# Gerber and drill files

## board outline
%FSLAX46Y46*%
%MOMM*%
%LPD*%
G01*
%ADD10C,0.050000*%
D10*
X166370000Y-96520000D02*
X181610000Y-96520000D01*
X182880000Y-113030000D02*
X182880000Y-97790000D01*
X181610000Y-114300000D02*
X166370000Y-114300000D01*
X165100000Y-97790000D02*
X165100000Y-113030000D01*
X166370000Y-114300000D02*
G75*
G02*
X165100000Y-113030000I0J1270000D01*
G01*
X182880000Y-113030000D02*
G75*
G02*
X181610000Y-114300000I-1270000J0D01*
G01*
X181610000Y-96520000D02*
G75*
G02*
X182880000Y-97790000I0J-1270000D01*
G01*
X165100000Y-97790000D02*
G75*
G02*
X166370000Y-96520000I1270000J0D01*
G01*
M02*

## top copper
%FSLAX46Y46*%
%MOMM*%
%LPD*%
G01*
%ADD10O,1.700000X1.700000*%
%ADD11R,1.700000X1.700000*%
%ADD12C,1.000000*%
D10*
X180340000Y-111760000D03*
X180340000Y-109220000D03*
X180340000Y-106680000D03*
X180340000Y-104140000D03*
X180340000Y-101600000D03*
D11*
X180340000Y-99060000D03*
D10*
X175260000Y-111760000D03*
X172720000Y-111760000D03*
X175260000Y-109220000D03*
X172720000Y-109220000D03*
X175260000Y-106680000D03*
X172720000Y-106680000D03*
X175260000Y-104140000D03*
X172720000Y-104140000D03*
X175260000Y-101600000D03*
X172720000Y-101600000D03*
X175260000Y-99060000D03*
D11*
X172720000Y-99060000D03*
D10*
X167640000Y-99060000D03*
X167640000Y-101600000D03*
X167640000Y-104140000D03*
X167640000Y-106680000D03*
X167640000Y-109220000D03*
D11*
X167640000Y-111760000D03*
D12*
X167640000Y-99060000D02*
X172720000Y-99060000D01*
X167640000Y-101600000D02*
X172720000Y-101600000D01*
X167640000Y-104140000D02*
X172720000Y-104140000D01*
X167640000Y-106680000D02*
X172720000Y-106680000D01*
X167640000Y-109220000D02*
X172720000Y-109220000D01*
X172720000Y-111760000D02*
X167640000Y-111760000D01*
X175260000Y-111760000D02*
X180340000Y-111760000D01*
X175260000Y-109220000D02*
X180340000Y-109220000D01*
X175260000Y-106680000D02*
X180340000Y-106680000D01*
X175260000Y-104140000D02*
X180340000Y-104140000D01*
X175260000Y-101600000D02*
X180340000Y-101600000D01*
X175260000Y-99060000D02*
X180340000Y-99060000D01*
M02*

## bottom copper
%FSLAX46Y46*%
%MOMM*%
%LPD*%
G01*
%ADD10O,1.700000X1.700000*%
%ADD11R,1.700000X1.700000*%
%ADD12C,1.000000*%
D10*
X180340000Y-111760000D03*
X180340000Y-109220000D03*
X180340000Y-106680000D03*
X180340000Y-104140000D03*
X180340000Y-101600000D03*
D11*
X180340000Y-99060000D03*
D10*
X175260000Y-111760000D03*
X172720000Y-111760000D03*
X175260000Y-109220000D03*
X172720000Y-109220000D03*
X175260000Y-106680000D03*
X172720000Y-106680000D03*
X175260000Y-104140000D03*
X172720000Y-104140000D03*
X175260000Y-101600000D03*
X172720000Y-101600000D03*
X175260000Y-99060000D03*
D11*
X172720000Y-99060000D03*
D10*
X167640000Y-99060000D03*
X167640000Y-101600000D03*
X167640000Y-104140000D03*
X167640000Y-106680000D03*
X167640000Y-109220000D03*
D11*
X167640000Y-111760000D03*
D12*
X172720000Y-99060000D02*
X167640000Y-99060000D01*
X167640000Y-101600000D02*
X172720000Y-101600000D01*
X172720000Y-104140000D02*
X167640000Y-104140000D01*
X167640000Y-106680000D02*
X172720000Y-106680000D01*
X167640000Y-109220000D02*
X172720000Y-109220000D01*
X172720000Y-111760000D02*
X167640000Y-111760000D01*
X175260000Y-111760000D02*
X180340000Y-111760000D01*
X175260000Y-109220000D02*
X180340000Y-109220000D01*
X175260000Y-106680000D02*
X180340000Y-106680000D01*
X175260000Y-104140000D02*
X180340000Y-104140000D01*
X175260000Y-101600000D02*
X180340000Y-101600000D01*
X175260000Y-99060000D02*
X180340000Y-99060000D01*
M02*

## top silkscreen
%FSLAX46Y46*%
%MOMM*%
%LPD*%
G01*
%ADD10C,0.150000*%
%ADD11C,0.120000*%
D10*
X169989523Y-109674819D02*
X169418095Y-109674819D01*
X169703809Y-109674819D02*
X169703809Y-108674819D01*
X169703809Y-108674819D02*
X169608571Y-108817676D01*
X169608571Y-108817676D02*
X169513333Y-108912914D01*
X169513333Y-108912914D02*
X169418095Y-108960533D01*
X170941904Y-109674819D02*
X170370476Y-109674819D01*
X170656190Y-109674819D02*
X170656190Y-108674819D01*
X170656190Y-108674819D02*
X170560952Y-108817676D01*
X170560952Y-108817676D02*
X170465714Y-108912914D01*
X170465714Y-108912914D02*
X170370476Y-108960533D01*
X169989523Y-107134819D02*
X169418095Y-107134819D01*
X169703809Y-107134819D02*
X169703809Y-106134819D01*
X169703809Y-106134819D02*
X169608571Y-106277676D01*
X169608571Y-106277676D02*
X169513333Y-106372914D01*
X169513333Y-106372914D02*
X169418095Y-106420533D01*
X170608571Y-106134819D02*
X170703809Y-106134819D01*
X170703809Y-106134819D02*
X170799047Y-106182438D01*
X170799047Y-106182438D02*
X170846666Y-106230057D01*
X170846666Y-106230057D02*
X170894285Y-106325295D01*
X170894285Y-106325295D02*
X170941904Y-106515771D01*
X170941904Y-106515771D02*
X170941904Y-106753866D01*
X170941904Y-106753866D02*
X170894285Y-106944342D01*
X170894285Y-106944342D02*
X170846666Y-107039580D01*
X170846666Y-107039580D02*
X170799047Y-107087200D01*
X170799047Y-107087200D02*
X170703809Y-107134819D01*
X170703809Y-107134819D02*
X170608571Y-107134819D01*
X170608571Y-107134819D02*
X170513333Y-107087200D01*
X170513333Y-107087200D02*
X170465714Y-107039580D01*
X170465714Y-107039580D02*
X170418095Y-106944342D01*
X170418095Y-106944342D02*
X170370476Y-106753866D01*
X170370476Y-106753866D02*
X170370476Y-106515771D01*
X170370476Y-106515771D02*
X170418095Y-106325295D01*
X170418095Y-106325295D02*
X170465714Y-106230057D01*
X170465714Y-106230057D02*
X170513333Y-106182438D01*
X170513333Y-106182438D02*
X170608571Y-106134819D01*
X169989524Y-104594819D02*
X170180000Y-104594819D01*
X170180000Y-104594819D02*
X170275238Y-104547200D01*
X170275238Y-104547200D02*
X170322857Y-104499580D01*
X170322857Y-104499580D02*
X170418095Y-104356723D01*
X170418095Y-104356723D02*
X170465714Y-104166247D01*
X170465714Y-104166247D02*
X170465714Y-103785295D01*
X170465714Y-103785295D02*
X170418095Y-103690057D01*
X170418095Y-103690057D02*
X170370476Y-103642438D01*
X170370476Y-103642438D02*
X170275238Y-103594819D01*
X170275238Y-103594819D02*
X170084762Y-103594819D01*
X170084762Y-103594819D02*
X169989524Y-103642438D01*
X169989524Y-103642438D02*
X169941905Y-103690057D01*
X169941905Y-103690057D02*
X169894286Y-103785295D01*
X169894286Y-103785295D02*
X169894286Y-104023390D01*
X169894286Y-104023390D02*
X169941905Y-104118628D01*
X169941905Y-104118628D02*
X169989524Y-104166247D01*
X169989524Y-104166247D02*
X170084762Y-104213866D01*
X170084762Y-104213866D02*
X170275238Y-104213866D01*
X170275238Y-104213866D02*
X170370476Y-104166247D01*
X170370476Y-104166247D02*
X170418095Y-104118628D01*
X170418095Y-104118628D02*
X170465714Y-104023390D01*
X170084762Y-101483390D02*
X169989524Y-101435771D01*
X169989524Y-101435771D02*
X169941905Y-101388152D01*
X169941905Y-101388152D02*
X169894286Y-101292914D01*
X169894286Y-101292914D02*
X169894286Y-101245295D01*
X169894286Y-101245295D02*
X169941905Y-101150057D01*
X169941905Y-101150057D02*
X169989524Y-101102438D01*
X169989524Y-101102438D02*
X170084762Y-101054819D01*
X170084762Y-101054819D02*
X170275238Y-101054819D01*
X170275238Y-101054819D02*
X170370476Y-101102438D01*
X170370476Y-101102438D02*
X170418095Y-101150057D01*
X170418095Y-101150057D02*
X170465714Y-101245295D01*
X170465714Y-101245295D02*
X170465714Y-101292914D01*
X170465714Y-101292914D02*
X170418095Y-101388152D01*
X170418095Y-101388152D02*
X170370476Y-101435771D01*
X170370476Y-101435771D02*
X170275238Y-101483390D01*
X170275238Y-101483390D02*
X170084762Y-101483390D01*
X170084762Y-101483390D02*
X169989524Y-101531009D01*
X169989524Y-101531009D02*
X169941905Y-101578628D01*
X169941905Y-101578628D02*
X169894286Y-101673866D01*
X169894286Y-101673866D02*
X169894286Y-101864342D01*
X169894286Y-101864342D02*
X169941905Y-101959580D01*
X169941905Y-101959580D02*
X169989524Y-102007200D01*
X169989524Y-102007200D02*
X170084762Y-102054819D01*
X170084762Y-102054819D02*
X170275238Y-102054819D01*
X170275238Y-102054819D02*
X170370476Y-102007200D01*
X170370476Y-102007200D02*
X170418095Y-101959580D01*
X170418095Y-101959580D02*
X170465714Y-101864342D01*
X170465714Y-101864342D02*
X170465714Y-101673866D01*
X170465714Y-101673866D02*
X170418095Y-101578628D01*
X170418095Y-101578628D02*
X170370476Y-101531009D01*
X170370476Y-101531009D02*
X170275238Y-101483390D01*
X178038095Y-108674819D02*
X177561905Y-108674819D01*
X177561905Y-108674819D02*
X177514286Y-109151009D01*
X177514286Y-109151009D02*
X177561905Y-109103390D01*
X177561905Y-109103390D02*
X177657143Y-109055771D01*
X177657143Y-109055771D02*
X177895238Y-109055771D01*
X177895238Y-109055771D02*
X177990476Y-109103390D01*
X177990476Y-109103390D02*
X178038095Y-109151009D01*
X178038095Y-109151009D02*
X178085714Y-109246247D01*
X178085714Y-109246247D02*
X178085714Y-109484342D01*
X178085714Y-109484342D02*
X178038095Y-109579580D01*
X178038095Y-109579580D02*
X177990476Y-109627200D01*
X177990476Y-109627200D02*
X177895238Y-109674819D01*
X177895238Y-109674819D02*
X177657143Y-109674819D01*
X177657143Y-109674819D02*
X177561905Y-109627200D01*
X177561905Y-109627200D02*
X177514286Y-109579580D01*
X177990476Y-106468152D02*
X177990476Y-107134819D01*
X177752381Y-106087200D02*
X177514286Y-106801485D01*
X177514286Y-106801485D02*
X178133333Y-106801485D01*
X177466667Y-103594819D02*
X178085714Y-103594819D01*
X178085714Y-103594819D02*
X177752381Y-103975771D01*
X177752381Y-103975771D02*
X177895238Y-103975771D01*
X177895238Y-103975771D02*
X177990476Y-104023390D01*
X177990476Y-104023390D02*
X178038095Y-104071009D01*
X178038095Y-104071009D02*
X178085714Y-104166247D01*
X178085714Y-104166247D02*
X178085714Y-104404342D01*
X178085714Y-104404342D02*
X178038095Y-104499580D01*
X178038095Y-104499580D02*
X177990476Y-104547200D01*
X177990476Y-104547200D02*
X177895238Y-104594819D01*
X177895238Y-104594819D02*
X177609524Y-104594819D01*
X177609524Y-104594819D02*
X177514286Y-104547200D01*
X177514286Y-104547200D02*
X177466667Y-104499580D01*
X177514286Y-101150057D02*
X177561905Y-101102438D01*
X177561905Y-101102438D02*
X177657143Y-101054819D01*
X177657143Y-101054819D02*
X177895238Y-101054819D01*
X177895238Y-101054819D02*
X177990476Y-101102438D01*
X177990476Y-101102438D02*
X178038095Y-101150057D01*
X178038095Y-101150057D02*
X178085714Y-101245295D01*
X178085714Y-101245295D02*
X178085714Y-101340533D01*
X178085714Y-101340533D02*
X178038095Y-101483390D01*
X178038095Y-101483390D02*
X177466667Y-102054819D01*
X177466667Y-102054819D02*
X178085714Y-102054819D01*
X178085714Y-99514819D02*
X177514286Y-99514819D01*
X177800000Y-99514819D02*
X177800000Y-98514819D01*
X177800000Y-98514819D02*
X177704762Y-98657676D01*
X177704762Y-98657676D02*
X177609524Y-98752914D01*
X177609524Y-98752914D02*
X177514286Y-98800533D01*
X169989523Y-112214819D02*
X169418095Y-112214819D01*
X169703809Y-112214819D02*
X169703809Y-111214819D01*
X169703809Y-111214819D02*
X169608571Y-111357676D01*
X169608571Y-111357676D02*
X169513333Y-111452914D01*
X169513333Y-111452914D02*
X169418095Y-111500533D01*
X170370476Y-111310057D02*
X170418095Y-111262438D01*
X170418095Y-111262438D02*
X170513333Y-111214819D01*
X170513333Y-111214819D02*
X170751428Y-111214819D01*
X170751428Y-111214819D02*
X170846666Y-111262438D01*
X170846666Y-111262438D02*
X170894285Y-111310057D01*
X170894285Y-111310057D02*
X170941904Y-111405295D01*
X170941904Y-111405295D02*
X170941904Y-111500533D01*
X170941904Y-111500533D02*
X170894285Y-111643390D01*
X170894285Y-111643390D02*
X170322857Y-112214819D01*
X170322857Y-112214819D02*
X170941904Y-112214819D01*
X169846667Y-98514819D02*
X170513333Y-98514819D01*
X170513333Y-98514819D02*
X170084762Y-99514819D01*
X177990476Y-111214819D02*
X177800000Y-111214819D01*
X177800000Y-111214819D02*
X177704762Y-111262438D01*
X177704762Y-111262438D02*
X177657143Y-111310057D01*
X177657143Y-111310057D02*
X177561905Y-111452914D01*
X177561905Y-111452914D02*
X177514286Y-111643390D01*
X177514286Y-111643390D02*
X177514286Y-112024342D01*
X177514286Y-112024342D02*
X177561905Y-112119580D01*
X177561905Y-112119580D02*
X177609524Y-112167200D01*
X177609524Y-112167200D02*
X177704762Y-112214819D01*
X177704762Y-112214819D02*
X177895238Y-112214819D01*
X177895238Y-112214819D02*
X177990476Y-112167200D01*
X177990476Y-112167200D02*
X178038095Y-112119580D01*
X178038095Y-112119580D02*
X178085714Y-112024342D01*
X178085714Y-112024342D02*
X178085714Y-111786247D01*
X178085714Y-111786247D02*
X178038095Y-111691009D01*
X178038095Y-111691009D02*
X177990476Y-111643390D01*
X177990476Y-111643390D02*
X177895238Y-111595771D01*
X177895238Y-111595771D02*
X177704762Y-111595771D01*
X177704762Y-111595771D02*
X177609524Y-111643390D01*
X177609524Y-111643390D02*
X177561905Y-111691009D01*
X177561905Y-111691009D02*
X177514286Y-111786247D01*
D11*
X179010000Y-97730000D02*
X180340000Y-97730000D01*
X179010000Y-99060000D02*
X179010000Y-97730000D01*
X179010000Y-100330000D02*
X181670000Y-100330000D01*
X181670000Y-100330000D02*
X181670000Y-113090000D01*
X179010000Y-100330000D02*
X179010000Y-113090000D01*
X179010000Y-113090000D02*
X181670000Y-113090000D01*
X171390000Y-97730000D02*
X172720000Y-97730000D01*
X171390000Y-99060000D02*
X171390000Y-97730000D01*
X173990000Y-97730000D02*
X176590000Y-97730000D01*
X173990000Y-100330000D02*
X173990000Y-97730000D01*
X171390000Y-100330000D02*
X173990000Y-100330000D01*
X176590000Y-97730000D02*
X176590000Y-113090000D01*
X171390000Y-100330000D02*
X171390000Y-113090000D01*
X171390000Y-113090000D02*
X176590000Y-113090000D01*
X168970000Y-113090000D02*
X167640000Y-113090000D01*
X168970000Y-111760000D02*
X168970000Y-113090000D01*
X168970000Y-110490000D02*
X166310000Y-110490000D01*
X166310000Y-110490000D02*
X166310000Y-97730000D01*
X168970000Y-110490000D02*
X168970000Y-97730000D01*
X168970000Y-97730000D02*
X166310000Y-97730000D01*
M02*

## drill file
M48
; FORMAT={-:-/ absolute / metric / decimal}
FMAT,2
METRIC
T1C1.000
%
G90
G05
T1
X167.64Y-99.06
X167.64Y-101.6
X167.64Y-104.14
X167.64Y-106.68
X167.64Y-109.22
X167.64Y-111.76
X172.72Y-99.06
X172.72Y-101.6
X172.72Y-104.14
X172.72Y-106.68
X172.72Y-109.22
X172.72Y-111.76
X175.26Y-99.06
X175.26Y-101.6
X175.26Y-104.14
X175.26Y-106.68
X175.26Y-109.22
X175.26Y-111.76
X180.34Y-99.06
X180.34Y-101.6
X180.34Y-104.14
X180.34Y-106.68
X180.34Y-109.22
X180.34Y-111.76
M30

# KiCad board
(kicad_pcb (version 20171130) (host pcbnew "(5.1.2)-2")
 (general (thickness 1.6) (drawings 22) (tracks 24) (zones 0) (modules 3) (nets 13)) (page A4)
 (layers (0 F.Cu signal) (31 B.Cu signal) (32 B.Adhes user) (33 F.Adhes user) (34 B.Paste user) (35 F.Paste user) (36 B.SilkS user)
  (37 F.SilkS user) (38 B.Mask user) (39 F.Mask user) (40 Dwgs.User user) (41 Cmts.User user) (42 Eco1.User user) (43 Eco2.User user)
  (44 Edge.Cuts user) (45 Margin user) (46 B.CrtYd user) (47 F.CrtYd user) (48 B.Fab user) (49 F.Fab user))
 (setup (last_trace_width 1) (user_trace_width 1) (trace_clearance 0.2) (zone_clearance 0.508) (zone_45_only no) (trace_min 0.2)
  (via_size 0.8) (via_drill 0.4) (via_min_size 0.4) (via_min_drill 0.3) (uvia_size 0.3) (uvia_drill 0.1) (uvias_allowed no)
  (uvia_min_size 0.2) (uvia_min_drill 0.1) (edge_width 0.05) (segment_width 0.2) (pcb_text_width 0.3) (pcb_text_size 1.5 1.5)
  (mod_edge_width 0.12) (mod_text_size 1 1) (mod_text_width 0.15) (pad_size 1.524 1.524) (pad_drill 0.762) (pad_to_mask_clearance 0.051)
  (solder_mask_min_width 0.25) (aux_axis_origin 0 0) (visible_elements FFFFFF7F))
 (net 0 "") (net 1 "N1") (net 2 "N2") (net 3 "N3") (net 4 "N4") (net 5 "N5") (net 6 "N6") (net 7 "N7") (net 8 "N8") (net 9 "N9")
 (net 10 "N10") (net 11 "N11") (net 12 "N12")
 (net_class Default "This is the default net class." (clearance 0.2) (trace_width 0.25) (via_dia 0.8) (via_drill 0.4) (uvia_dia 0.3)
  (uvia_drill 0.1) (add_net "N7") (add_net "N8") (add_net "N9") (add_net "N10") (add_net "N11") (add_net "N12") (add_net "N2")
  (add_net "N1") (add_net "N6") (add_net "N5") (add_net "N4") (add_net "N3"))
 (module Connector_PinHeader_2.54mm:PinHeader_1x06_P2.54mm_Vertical (layer F.Cu) (at 180.34 99.06)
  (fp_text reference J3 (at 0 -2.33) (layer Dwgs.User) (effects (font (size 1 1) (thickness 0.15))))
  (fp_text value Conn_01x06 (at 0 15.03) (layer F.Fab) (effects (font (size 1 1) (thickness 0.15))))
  (fp_line (start -1.33 -1.33) (end 0 -1.33) (layer F.SilkS) (width 0.12))
  (fp_line (start -1.33 0) (end -1.33 -1.33) (layer F.SilkS) (width 0.12))
  (fp_line (start -1.33 1.27) (end 1.33 1.27) (layer F.SilkS) (width 0.12))
  (fp_line (start 1.33 1.27) (end 1.33 14.03) (layer F.SilkS) (width 0.12))
  (fp_line (start -1.33 1.27) (end -1.33 14.03) (layer F.SilkS) (width 0.12))
  (fp_line (start -1.33 14.03) (end 1.33 14.03) (layer F.SilkS) (width 0.12))
  (pad 6 thru_hole oval (at 0 12.7) (size 1.7 1.7) (drill 1) (layers *.Cu *.Mask) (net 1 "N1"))
  (pad 5 thru_hole oval (at 0 10.16) (size 1.7 1.7) (drill 1) (layers *.Cu *.Mask) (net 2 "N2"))
  (pad 4 thru_hole oval (at 0 7.62) (size 1.7 1.7) (drill 1) (layers *.Cu *.Mask) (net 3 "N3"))
  (pad 3 thru_hole oval (at 0 5.08) (size 1.7 1.7) (drill 1) (layers *.Cu *.Mask) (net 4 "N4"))
  (pad 2 thru_hole oval (at 0 2.54) (size 1.7 1.7) (drill 1) (layers *.Cu *.Mask) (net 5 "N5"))
  (pad 1 thru_hole rect (at 0 0) (size 1.7 1.7) (drill 1) (layers *.Cu *.Mask) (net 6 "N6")))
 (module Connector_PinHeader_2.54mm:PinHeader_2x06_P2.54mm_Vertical (layer F.Cu) (at 172.72 99.06)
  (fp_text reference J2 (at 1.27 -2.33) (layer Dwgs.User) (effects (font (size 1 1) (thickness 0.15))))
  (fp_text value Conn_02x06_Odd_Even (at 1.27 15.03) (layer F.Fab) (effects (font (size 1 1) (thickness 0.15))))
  (fp_line (start -1.33 -1.33) (end 0 -1.33) (layer F.SilkS) (width 0.12))
  (fp_line (start -1.33 0) (end -1.33 -1.33) (layer F.SilkS) (width 0.12))
  (fp_line (start 1.27 -1.33) (end 3.87 -1.33) (layer F.SilkS) (width 0.12))
  (fp_line (start 1.27 1.27) (end 1.27 -1.33) (layer F.SilkS) (width 0.12))
  (fp_line (start -1.33 1.27) (end 1.27 1.27) (layer F.SilkS) (width 0.12))
  (fp_line (start 3.87 -1.33) (end 3.87 14.03) (layer F.SilkS) (width 0.12))
  (fp_line (start -1.33 1.27) (end -1.33 14.03) (layer F.SilkS) (width 0.12))
  (fp_line (start -1.33 14.03) (end 3.87 14.03) (layer F.SilkS) (width 0.12))
  (pad 12 thru_hole oval (at 2.54 12.7) (size 1.7 1.7) (drill 1) (layers *.Cu *.Mask) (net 1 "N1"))
  (pad 11 thru_hole oval (at 0 12.7) (size 1.7 1.7) (drill 1) (layers *.Cu *.Mask) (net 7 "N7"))
  (pad 10 thru_hole oval (at 2.54 10.16) (size 1.7 1.7) (drill 1) (layers *.Cu *.Mask) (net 2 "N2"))
  (pad 9 thru_hole oval (at 0 10.16) (size 1.7 1.7) (drill 1) (layers *.Cu *.Mask) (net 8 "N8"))
  (pad 8 thru_hole oval (at 2.54 7.62) (size 1.7 1.7) (drill 1) (layers *.Cu *.Mask) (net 3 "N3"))
  (pad 7 thru_hole oval (at 0 7.62) (size 1.7 1.7) (drill 1) (layers *.Cu *.Mask) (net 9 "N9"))
  (pad 6 thru_hole oval (at 2.54 5.08) (size 1.7 1.7) (drill 1) (layers *.Cu *.Mask) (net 4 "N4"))
  (pad 5 thru_hole oval (at 0 5.08) (size 1.7 1.7) (drill 1) (layers *.Cu *.Mask) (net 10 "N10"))
  (pad 4 thru_hole oval (at 2.54 2.54) (size 1.7 1.7) (drill 1) (layers *.Cu *.Mask) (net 5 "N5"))
  (pad 3 thru_hole oval (at 0 2.54) (size 1.7 1.7) (drill 1) (layers *.Cu *.Mask) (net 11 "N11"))
  (pad 2 thru_hole oval (at 2.54 0) (size 1.7 1.7) (drill 1) (layers *.Cu *.Mask) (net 6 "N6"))
  (pad 1 thru_hole rect (at 0 0) (size 1.7 1.7) (drill 1) (layers *.Cu *.Mask) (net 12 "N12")))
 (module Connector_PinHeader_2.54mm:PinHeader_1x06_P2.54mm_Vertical (layer F.Cu) (at 167.64 111.76 180)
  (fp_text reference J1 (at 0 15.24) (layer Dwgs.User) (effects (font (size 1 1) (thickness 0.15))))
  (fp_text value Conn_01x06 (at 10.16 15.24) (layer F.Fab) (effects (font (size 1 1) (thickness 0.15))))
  (fp_line (start -1.33 -1.33) (end 0 -1.33) (layer F.SilkS) (width 0.12))
  (fp_line (start -1.33 0) (end -1.33 -1.33) (layer F.SilkS) (width 0.12))
  (fp_line (start -1.33 1.27) (end 1.33 1.27) (layer F.SilkS) (width 0.12))
  (fp_line (start 1.33 1.27) (end 1.33 14.03) (layer F.SilkS) (width 0.12))
  (fp_line (start -1.33 1.27) (end -1.33 14.03) (layer F.SilkS) (width 0.12))
  (fp_line (start -1.33 14.03) (end 1.33 14.03) (layer F.SilkS) (width 0.12))
  (pad 6 thru_hole oval (at 0 12.7 180) (size 1.7 1.7) (drill 1) (layers *.Cu *.Mask) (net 12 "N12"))
  (pad 5 thru_hole oval (at 0 10.16 180) (size 1.7 1.7) (drill 1) (layers *.Cu *.Mask) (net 11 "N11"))
  (pad 4 thru_hole oval (at 0 7.62 180) (size 1.7 1.7) (drill 1) (layers *.Cu *.Mask) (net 10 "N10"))
  (pad 3 thru_hole oval (at 0 5.08 180) (size 1.7 1.7) (drill 1) (layers *.Cu *.Mask) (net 9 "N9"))
  (pad 2 thru_hole oval (at 0 2.54 180) (size 1.7 1.7) (drill 1) (layers *.Cu *.Mask) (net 8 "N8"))
  (pad 1 thru_hole rect (at 0 0 180) (size 1.7 1.7) (drill 1) (layers *.Cu *.Mask) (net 7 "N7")))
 (gr_line (start 166.37 96.52) (end 181.61 96.52) (layer Edge.Cuts) (width 0.05))
 (gr_line (start 182.88 113.03) (end 182.88 97.79) (layer Edge.Cuts) (width 0.05))
 (gr_line (start 181.61 114.3) (end 166.37 114.3) (layer Edge.Cuts) (width 0.05))
 (gr_line (start 165.1 97.79) (end 165.1 113.03) (layer Edge.Cuts) (width 0.05))
 (gr_arc (start 166.37 113.03) (end 165.1 113.03) (angle -90) (layer Edge.Cuts) (width 0.05))
 (gr_arc (start 181.61 113.03) (end 181.61 114.3) (angle -90) (layer Edge.Cuts) (width 0.05))
 (gr_arc (start 181.61 97.79) (end 182.88 97.79) (angle -90) (layer Edge.Cuts) (width 0.05))
 (gr_arc (start 166.37 97.79) (end 166.37 96.52) (angle -90) (layer Edge.Cuts) (width 0.05))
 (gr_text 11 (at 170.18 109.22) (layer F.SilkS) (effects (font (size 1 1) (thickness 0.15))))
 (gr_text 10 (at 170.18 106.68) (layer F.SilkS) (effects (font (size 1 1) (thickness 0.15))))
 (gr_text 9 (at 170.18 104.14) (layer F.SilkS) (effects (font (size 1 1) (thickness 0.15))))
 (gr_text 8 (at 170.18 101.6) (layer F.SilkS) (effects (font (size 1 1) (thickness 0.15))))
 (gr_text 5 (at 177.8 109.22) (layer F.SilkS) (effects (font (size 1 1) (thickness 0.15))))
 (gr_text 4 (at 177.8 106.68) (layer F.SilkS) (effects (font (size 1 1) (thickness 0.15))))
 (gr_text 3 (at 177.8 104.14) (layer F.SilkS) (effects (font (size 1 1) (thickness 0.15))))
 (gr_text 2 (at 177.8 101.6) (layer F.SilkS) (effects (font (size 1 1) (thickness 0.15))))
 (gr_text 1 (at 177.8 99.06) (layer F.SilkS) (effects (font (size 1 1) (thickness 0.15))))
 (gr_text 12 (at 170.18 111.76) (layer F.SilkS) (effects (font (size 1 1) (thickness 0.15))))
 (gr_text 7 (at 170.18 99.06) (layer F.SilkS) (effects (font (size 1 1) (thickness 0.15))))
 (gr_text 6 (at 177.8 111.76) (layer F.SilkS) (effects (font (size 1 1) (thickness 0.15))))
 (segment (start 167.64 99.06) (end 172.72 99.06) (width 1) (layer F.Cu) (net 12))
 (segment (start 172.72 99.06) (end 167.64 99.06) (width 1) (layer B.Cu) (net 12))
 (segment (start 167.64 101.6) (end 172.72 101.6) (width 1) (layer F.Cu) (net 11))
 (segment (start 167.64 101.6) (end 172.72 101.6) (width 1) (layer B.Cu) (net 11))
 (segment (start 167.64 104.14) (end 172.72 104.14) (width 1) (layer F.Cu) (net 10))
 (segment (start 172.72 104.14) (end 167.64 104.14) (width 1) (layer B.Cu) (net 10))
 (segment (start 167.64 106.68) (end 172.72 106.68) (width 1) (layer F.Cu) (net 9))
 (segment (start 167.64 106.68) (end 172.72 106.68) (width 1) (layer B.Cu) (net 9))
 (segment (start 167.64 109.22) (end 172.72 109.22) (width 1) (layer F.Cu) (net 8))
 (segment (start 167.64 109.22) (end 172.72 109.22) (width 1) (layer B.Cu) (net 8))
 (segment (start 172.72 111.76) (end 167.64 111.76) (width 1) (layer F.Cu) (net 7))
 (segment (start 172.72 111.76) (end 167.64 111.76) (width 1) (layer B.Cu) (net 7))
 (segment (start 175.26 111.76) (end 180.34 111.76) (width 1) (layer F.Cu) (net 1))
 (segment (start 175.26 111.76) (end 180.34 111.76) (width 1) (layer B.Cu) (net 1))
 (segment (start 175.26 109.22) (end 180.34 109.22) (width 1) (layer B.Cu) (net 2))
 (segment (start 175.26 109.22) (end 180.34 109.22) (width 1) (layer F.Cu) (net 2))
 (segment (start 175.26 106.68) (end 180.34 106.68) (width 1) (layer F.Cu) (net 3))
 (segment (start 175.26 106.68) (end 180.34 106.68) (width 1) (layer B.Cu) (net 3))
 (segment (start 175.26 104.14) (end 180.34 104.14) (width 1) (layer F.Cu) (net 4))
 (segment (start 175.26 104.14) (end 180.34 104.14) (width 1) (layer B.Cu) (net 4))
 (segment (start 175.26 101.6) (end 180.34 101.6) (width 1) (layer F.Cu) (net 5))
 (segment (start 175.26 101.6) (end 180.34 101.6) (width 1) (layer B.Cu) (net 5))
 (segment (start 175.26 99.06) (end 180.34 99.06) (width 1) (layer F.Cu) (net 6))
 (segment (start 175.26 99.06) (end 180.34 99.06) (width 1) (layer B.Cu) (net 6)))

